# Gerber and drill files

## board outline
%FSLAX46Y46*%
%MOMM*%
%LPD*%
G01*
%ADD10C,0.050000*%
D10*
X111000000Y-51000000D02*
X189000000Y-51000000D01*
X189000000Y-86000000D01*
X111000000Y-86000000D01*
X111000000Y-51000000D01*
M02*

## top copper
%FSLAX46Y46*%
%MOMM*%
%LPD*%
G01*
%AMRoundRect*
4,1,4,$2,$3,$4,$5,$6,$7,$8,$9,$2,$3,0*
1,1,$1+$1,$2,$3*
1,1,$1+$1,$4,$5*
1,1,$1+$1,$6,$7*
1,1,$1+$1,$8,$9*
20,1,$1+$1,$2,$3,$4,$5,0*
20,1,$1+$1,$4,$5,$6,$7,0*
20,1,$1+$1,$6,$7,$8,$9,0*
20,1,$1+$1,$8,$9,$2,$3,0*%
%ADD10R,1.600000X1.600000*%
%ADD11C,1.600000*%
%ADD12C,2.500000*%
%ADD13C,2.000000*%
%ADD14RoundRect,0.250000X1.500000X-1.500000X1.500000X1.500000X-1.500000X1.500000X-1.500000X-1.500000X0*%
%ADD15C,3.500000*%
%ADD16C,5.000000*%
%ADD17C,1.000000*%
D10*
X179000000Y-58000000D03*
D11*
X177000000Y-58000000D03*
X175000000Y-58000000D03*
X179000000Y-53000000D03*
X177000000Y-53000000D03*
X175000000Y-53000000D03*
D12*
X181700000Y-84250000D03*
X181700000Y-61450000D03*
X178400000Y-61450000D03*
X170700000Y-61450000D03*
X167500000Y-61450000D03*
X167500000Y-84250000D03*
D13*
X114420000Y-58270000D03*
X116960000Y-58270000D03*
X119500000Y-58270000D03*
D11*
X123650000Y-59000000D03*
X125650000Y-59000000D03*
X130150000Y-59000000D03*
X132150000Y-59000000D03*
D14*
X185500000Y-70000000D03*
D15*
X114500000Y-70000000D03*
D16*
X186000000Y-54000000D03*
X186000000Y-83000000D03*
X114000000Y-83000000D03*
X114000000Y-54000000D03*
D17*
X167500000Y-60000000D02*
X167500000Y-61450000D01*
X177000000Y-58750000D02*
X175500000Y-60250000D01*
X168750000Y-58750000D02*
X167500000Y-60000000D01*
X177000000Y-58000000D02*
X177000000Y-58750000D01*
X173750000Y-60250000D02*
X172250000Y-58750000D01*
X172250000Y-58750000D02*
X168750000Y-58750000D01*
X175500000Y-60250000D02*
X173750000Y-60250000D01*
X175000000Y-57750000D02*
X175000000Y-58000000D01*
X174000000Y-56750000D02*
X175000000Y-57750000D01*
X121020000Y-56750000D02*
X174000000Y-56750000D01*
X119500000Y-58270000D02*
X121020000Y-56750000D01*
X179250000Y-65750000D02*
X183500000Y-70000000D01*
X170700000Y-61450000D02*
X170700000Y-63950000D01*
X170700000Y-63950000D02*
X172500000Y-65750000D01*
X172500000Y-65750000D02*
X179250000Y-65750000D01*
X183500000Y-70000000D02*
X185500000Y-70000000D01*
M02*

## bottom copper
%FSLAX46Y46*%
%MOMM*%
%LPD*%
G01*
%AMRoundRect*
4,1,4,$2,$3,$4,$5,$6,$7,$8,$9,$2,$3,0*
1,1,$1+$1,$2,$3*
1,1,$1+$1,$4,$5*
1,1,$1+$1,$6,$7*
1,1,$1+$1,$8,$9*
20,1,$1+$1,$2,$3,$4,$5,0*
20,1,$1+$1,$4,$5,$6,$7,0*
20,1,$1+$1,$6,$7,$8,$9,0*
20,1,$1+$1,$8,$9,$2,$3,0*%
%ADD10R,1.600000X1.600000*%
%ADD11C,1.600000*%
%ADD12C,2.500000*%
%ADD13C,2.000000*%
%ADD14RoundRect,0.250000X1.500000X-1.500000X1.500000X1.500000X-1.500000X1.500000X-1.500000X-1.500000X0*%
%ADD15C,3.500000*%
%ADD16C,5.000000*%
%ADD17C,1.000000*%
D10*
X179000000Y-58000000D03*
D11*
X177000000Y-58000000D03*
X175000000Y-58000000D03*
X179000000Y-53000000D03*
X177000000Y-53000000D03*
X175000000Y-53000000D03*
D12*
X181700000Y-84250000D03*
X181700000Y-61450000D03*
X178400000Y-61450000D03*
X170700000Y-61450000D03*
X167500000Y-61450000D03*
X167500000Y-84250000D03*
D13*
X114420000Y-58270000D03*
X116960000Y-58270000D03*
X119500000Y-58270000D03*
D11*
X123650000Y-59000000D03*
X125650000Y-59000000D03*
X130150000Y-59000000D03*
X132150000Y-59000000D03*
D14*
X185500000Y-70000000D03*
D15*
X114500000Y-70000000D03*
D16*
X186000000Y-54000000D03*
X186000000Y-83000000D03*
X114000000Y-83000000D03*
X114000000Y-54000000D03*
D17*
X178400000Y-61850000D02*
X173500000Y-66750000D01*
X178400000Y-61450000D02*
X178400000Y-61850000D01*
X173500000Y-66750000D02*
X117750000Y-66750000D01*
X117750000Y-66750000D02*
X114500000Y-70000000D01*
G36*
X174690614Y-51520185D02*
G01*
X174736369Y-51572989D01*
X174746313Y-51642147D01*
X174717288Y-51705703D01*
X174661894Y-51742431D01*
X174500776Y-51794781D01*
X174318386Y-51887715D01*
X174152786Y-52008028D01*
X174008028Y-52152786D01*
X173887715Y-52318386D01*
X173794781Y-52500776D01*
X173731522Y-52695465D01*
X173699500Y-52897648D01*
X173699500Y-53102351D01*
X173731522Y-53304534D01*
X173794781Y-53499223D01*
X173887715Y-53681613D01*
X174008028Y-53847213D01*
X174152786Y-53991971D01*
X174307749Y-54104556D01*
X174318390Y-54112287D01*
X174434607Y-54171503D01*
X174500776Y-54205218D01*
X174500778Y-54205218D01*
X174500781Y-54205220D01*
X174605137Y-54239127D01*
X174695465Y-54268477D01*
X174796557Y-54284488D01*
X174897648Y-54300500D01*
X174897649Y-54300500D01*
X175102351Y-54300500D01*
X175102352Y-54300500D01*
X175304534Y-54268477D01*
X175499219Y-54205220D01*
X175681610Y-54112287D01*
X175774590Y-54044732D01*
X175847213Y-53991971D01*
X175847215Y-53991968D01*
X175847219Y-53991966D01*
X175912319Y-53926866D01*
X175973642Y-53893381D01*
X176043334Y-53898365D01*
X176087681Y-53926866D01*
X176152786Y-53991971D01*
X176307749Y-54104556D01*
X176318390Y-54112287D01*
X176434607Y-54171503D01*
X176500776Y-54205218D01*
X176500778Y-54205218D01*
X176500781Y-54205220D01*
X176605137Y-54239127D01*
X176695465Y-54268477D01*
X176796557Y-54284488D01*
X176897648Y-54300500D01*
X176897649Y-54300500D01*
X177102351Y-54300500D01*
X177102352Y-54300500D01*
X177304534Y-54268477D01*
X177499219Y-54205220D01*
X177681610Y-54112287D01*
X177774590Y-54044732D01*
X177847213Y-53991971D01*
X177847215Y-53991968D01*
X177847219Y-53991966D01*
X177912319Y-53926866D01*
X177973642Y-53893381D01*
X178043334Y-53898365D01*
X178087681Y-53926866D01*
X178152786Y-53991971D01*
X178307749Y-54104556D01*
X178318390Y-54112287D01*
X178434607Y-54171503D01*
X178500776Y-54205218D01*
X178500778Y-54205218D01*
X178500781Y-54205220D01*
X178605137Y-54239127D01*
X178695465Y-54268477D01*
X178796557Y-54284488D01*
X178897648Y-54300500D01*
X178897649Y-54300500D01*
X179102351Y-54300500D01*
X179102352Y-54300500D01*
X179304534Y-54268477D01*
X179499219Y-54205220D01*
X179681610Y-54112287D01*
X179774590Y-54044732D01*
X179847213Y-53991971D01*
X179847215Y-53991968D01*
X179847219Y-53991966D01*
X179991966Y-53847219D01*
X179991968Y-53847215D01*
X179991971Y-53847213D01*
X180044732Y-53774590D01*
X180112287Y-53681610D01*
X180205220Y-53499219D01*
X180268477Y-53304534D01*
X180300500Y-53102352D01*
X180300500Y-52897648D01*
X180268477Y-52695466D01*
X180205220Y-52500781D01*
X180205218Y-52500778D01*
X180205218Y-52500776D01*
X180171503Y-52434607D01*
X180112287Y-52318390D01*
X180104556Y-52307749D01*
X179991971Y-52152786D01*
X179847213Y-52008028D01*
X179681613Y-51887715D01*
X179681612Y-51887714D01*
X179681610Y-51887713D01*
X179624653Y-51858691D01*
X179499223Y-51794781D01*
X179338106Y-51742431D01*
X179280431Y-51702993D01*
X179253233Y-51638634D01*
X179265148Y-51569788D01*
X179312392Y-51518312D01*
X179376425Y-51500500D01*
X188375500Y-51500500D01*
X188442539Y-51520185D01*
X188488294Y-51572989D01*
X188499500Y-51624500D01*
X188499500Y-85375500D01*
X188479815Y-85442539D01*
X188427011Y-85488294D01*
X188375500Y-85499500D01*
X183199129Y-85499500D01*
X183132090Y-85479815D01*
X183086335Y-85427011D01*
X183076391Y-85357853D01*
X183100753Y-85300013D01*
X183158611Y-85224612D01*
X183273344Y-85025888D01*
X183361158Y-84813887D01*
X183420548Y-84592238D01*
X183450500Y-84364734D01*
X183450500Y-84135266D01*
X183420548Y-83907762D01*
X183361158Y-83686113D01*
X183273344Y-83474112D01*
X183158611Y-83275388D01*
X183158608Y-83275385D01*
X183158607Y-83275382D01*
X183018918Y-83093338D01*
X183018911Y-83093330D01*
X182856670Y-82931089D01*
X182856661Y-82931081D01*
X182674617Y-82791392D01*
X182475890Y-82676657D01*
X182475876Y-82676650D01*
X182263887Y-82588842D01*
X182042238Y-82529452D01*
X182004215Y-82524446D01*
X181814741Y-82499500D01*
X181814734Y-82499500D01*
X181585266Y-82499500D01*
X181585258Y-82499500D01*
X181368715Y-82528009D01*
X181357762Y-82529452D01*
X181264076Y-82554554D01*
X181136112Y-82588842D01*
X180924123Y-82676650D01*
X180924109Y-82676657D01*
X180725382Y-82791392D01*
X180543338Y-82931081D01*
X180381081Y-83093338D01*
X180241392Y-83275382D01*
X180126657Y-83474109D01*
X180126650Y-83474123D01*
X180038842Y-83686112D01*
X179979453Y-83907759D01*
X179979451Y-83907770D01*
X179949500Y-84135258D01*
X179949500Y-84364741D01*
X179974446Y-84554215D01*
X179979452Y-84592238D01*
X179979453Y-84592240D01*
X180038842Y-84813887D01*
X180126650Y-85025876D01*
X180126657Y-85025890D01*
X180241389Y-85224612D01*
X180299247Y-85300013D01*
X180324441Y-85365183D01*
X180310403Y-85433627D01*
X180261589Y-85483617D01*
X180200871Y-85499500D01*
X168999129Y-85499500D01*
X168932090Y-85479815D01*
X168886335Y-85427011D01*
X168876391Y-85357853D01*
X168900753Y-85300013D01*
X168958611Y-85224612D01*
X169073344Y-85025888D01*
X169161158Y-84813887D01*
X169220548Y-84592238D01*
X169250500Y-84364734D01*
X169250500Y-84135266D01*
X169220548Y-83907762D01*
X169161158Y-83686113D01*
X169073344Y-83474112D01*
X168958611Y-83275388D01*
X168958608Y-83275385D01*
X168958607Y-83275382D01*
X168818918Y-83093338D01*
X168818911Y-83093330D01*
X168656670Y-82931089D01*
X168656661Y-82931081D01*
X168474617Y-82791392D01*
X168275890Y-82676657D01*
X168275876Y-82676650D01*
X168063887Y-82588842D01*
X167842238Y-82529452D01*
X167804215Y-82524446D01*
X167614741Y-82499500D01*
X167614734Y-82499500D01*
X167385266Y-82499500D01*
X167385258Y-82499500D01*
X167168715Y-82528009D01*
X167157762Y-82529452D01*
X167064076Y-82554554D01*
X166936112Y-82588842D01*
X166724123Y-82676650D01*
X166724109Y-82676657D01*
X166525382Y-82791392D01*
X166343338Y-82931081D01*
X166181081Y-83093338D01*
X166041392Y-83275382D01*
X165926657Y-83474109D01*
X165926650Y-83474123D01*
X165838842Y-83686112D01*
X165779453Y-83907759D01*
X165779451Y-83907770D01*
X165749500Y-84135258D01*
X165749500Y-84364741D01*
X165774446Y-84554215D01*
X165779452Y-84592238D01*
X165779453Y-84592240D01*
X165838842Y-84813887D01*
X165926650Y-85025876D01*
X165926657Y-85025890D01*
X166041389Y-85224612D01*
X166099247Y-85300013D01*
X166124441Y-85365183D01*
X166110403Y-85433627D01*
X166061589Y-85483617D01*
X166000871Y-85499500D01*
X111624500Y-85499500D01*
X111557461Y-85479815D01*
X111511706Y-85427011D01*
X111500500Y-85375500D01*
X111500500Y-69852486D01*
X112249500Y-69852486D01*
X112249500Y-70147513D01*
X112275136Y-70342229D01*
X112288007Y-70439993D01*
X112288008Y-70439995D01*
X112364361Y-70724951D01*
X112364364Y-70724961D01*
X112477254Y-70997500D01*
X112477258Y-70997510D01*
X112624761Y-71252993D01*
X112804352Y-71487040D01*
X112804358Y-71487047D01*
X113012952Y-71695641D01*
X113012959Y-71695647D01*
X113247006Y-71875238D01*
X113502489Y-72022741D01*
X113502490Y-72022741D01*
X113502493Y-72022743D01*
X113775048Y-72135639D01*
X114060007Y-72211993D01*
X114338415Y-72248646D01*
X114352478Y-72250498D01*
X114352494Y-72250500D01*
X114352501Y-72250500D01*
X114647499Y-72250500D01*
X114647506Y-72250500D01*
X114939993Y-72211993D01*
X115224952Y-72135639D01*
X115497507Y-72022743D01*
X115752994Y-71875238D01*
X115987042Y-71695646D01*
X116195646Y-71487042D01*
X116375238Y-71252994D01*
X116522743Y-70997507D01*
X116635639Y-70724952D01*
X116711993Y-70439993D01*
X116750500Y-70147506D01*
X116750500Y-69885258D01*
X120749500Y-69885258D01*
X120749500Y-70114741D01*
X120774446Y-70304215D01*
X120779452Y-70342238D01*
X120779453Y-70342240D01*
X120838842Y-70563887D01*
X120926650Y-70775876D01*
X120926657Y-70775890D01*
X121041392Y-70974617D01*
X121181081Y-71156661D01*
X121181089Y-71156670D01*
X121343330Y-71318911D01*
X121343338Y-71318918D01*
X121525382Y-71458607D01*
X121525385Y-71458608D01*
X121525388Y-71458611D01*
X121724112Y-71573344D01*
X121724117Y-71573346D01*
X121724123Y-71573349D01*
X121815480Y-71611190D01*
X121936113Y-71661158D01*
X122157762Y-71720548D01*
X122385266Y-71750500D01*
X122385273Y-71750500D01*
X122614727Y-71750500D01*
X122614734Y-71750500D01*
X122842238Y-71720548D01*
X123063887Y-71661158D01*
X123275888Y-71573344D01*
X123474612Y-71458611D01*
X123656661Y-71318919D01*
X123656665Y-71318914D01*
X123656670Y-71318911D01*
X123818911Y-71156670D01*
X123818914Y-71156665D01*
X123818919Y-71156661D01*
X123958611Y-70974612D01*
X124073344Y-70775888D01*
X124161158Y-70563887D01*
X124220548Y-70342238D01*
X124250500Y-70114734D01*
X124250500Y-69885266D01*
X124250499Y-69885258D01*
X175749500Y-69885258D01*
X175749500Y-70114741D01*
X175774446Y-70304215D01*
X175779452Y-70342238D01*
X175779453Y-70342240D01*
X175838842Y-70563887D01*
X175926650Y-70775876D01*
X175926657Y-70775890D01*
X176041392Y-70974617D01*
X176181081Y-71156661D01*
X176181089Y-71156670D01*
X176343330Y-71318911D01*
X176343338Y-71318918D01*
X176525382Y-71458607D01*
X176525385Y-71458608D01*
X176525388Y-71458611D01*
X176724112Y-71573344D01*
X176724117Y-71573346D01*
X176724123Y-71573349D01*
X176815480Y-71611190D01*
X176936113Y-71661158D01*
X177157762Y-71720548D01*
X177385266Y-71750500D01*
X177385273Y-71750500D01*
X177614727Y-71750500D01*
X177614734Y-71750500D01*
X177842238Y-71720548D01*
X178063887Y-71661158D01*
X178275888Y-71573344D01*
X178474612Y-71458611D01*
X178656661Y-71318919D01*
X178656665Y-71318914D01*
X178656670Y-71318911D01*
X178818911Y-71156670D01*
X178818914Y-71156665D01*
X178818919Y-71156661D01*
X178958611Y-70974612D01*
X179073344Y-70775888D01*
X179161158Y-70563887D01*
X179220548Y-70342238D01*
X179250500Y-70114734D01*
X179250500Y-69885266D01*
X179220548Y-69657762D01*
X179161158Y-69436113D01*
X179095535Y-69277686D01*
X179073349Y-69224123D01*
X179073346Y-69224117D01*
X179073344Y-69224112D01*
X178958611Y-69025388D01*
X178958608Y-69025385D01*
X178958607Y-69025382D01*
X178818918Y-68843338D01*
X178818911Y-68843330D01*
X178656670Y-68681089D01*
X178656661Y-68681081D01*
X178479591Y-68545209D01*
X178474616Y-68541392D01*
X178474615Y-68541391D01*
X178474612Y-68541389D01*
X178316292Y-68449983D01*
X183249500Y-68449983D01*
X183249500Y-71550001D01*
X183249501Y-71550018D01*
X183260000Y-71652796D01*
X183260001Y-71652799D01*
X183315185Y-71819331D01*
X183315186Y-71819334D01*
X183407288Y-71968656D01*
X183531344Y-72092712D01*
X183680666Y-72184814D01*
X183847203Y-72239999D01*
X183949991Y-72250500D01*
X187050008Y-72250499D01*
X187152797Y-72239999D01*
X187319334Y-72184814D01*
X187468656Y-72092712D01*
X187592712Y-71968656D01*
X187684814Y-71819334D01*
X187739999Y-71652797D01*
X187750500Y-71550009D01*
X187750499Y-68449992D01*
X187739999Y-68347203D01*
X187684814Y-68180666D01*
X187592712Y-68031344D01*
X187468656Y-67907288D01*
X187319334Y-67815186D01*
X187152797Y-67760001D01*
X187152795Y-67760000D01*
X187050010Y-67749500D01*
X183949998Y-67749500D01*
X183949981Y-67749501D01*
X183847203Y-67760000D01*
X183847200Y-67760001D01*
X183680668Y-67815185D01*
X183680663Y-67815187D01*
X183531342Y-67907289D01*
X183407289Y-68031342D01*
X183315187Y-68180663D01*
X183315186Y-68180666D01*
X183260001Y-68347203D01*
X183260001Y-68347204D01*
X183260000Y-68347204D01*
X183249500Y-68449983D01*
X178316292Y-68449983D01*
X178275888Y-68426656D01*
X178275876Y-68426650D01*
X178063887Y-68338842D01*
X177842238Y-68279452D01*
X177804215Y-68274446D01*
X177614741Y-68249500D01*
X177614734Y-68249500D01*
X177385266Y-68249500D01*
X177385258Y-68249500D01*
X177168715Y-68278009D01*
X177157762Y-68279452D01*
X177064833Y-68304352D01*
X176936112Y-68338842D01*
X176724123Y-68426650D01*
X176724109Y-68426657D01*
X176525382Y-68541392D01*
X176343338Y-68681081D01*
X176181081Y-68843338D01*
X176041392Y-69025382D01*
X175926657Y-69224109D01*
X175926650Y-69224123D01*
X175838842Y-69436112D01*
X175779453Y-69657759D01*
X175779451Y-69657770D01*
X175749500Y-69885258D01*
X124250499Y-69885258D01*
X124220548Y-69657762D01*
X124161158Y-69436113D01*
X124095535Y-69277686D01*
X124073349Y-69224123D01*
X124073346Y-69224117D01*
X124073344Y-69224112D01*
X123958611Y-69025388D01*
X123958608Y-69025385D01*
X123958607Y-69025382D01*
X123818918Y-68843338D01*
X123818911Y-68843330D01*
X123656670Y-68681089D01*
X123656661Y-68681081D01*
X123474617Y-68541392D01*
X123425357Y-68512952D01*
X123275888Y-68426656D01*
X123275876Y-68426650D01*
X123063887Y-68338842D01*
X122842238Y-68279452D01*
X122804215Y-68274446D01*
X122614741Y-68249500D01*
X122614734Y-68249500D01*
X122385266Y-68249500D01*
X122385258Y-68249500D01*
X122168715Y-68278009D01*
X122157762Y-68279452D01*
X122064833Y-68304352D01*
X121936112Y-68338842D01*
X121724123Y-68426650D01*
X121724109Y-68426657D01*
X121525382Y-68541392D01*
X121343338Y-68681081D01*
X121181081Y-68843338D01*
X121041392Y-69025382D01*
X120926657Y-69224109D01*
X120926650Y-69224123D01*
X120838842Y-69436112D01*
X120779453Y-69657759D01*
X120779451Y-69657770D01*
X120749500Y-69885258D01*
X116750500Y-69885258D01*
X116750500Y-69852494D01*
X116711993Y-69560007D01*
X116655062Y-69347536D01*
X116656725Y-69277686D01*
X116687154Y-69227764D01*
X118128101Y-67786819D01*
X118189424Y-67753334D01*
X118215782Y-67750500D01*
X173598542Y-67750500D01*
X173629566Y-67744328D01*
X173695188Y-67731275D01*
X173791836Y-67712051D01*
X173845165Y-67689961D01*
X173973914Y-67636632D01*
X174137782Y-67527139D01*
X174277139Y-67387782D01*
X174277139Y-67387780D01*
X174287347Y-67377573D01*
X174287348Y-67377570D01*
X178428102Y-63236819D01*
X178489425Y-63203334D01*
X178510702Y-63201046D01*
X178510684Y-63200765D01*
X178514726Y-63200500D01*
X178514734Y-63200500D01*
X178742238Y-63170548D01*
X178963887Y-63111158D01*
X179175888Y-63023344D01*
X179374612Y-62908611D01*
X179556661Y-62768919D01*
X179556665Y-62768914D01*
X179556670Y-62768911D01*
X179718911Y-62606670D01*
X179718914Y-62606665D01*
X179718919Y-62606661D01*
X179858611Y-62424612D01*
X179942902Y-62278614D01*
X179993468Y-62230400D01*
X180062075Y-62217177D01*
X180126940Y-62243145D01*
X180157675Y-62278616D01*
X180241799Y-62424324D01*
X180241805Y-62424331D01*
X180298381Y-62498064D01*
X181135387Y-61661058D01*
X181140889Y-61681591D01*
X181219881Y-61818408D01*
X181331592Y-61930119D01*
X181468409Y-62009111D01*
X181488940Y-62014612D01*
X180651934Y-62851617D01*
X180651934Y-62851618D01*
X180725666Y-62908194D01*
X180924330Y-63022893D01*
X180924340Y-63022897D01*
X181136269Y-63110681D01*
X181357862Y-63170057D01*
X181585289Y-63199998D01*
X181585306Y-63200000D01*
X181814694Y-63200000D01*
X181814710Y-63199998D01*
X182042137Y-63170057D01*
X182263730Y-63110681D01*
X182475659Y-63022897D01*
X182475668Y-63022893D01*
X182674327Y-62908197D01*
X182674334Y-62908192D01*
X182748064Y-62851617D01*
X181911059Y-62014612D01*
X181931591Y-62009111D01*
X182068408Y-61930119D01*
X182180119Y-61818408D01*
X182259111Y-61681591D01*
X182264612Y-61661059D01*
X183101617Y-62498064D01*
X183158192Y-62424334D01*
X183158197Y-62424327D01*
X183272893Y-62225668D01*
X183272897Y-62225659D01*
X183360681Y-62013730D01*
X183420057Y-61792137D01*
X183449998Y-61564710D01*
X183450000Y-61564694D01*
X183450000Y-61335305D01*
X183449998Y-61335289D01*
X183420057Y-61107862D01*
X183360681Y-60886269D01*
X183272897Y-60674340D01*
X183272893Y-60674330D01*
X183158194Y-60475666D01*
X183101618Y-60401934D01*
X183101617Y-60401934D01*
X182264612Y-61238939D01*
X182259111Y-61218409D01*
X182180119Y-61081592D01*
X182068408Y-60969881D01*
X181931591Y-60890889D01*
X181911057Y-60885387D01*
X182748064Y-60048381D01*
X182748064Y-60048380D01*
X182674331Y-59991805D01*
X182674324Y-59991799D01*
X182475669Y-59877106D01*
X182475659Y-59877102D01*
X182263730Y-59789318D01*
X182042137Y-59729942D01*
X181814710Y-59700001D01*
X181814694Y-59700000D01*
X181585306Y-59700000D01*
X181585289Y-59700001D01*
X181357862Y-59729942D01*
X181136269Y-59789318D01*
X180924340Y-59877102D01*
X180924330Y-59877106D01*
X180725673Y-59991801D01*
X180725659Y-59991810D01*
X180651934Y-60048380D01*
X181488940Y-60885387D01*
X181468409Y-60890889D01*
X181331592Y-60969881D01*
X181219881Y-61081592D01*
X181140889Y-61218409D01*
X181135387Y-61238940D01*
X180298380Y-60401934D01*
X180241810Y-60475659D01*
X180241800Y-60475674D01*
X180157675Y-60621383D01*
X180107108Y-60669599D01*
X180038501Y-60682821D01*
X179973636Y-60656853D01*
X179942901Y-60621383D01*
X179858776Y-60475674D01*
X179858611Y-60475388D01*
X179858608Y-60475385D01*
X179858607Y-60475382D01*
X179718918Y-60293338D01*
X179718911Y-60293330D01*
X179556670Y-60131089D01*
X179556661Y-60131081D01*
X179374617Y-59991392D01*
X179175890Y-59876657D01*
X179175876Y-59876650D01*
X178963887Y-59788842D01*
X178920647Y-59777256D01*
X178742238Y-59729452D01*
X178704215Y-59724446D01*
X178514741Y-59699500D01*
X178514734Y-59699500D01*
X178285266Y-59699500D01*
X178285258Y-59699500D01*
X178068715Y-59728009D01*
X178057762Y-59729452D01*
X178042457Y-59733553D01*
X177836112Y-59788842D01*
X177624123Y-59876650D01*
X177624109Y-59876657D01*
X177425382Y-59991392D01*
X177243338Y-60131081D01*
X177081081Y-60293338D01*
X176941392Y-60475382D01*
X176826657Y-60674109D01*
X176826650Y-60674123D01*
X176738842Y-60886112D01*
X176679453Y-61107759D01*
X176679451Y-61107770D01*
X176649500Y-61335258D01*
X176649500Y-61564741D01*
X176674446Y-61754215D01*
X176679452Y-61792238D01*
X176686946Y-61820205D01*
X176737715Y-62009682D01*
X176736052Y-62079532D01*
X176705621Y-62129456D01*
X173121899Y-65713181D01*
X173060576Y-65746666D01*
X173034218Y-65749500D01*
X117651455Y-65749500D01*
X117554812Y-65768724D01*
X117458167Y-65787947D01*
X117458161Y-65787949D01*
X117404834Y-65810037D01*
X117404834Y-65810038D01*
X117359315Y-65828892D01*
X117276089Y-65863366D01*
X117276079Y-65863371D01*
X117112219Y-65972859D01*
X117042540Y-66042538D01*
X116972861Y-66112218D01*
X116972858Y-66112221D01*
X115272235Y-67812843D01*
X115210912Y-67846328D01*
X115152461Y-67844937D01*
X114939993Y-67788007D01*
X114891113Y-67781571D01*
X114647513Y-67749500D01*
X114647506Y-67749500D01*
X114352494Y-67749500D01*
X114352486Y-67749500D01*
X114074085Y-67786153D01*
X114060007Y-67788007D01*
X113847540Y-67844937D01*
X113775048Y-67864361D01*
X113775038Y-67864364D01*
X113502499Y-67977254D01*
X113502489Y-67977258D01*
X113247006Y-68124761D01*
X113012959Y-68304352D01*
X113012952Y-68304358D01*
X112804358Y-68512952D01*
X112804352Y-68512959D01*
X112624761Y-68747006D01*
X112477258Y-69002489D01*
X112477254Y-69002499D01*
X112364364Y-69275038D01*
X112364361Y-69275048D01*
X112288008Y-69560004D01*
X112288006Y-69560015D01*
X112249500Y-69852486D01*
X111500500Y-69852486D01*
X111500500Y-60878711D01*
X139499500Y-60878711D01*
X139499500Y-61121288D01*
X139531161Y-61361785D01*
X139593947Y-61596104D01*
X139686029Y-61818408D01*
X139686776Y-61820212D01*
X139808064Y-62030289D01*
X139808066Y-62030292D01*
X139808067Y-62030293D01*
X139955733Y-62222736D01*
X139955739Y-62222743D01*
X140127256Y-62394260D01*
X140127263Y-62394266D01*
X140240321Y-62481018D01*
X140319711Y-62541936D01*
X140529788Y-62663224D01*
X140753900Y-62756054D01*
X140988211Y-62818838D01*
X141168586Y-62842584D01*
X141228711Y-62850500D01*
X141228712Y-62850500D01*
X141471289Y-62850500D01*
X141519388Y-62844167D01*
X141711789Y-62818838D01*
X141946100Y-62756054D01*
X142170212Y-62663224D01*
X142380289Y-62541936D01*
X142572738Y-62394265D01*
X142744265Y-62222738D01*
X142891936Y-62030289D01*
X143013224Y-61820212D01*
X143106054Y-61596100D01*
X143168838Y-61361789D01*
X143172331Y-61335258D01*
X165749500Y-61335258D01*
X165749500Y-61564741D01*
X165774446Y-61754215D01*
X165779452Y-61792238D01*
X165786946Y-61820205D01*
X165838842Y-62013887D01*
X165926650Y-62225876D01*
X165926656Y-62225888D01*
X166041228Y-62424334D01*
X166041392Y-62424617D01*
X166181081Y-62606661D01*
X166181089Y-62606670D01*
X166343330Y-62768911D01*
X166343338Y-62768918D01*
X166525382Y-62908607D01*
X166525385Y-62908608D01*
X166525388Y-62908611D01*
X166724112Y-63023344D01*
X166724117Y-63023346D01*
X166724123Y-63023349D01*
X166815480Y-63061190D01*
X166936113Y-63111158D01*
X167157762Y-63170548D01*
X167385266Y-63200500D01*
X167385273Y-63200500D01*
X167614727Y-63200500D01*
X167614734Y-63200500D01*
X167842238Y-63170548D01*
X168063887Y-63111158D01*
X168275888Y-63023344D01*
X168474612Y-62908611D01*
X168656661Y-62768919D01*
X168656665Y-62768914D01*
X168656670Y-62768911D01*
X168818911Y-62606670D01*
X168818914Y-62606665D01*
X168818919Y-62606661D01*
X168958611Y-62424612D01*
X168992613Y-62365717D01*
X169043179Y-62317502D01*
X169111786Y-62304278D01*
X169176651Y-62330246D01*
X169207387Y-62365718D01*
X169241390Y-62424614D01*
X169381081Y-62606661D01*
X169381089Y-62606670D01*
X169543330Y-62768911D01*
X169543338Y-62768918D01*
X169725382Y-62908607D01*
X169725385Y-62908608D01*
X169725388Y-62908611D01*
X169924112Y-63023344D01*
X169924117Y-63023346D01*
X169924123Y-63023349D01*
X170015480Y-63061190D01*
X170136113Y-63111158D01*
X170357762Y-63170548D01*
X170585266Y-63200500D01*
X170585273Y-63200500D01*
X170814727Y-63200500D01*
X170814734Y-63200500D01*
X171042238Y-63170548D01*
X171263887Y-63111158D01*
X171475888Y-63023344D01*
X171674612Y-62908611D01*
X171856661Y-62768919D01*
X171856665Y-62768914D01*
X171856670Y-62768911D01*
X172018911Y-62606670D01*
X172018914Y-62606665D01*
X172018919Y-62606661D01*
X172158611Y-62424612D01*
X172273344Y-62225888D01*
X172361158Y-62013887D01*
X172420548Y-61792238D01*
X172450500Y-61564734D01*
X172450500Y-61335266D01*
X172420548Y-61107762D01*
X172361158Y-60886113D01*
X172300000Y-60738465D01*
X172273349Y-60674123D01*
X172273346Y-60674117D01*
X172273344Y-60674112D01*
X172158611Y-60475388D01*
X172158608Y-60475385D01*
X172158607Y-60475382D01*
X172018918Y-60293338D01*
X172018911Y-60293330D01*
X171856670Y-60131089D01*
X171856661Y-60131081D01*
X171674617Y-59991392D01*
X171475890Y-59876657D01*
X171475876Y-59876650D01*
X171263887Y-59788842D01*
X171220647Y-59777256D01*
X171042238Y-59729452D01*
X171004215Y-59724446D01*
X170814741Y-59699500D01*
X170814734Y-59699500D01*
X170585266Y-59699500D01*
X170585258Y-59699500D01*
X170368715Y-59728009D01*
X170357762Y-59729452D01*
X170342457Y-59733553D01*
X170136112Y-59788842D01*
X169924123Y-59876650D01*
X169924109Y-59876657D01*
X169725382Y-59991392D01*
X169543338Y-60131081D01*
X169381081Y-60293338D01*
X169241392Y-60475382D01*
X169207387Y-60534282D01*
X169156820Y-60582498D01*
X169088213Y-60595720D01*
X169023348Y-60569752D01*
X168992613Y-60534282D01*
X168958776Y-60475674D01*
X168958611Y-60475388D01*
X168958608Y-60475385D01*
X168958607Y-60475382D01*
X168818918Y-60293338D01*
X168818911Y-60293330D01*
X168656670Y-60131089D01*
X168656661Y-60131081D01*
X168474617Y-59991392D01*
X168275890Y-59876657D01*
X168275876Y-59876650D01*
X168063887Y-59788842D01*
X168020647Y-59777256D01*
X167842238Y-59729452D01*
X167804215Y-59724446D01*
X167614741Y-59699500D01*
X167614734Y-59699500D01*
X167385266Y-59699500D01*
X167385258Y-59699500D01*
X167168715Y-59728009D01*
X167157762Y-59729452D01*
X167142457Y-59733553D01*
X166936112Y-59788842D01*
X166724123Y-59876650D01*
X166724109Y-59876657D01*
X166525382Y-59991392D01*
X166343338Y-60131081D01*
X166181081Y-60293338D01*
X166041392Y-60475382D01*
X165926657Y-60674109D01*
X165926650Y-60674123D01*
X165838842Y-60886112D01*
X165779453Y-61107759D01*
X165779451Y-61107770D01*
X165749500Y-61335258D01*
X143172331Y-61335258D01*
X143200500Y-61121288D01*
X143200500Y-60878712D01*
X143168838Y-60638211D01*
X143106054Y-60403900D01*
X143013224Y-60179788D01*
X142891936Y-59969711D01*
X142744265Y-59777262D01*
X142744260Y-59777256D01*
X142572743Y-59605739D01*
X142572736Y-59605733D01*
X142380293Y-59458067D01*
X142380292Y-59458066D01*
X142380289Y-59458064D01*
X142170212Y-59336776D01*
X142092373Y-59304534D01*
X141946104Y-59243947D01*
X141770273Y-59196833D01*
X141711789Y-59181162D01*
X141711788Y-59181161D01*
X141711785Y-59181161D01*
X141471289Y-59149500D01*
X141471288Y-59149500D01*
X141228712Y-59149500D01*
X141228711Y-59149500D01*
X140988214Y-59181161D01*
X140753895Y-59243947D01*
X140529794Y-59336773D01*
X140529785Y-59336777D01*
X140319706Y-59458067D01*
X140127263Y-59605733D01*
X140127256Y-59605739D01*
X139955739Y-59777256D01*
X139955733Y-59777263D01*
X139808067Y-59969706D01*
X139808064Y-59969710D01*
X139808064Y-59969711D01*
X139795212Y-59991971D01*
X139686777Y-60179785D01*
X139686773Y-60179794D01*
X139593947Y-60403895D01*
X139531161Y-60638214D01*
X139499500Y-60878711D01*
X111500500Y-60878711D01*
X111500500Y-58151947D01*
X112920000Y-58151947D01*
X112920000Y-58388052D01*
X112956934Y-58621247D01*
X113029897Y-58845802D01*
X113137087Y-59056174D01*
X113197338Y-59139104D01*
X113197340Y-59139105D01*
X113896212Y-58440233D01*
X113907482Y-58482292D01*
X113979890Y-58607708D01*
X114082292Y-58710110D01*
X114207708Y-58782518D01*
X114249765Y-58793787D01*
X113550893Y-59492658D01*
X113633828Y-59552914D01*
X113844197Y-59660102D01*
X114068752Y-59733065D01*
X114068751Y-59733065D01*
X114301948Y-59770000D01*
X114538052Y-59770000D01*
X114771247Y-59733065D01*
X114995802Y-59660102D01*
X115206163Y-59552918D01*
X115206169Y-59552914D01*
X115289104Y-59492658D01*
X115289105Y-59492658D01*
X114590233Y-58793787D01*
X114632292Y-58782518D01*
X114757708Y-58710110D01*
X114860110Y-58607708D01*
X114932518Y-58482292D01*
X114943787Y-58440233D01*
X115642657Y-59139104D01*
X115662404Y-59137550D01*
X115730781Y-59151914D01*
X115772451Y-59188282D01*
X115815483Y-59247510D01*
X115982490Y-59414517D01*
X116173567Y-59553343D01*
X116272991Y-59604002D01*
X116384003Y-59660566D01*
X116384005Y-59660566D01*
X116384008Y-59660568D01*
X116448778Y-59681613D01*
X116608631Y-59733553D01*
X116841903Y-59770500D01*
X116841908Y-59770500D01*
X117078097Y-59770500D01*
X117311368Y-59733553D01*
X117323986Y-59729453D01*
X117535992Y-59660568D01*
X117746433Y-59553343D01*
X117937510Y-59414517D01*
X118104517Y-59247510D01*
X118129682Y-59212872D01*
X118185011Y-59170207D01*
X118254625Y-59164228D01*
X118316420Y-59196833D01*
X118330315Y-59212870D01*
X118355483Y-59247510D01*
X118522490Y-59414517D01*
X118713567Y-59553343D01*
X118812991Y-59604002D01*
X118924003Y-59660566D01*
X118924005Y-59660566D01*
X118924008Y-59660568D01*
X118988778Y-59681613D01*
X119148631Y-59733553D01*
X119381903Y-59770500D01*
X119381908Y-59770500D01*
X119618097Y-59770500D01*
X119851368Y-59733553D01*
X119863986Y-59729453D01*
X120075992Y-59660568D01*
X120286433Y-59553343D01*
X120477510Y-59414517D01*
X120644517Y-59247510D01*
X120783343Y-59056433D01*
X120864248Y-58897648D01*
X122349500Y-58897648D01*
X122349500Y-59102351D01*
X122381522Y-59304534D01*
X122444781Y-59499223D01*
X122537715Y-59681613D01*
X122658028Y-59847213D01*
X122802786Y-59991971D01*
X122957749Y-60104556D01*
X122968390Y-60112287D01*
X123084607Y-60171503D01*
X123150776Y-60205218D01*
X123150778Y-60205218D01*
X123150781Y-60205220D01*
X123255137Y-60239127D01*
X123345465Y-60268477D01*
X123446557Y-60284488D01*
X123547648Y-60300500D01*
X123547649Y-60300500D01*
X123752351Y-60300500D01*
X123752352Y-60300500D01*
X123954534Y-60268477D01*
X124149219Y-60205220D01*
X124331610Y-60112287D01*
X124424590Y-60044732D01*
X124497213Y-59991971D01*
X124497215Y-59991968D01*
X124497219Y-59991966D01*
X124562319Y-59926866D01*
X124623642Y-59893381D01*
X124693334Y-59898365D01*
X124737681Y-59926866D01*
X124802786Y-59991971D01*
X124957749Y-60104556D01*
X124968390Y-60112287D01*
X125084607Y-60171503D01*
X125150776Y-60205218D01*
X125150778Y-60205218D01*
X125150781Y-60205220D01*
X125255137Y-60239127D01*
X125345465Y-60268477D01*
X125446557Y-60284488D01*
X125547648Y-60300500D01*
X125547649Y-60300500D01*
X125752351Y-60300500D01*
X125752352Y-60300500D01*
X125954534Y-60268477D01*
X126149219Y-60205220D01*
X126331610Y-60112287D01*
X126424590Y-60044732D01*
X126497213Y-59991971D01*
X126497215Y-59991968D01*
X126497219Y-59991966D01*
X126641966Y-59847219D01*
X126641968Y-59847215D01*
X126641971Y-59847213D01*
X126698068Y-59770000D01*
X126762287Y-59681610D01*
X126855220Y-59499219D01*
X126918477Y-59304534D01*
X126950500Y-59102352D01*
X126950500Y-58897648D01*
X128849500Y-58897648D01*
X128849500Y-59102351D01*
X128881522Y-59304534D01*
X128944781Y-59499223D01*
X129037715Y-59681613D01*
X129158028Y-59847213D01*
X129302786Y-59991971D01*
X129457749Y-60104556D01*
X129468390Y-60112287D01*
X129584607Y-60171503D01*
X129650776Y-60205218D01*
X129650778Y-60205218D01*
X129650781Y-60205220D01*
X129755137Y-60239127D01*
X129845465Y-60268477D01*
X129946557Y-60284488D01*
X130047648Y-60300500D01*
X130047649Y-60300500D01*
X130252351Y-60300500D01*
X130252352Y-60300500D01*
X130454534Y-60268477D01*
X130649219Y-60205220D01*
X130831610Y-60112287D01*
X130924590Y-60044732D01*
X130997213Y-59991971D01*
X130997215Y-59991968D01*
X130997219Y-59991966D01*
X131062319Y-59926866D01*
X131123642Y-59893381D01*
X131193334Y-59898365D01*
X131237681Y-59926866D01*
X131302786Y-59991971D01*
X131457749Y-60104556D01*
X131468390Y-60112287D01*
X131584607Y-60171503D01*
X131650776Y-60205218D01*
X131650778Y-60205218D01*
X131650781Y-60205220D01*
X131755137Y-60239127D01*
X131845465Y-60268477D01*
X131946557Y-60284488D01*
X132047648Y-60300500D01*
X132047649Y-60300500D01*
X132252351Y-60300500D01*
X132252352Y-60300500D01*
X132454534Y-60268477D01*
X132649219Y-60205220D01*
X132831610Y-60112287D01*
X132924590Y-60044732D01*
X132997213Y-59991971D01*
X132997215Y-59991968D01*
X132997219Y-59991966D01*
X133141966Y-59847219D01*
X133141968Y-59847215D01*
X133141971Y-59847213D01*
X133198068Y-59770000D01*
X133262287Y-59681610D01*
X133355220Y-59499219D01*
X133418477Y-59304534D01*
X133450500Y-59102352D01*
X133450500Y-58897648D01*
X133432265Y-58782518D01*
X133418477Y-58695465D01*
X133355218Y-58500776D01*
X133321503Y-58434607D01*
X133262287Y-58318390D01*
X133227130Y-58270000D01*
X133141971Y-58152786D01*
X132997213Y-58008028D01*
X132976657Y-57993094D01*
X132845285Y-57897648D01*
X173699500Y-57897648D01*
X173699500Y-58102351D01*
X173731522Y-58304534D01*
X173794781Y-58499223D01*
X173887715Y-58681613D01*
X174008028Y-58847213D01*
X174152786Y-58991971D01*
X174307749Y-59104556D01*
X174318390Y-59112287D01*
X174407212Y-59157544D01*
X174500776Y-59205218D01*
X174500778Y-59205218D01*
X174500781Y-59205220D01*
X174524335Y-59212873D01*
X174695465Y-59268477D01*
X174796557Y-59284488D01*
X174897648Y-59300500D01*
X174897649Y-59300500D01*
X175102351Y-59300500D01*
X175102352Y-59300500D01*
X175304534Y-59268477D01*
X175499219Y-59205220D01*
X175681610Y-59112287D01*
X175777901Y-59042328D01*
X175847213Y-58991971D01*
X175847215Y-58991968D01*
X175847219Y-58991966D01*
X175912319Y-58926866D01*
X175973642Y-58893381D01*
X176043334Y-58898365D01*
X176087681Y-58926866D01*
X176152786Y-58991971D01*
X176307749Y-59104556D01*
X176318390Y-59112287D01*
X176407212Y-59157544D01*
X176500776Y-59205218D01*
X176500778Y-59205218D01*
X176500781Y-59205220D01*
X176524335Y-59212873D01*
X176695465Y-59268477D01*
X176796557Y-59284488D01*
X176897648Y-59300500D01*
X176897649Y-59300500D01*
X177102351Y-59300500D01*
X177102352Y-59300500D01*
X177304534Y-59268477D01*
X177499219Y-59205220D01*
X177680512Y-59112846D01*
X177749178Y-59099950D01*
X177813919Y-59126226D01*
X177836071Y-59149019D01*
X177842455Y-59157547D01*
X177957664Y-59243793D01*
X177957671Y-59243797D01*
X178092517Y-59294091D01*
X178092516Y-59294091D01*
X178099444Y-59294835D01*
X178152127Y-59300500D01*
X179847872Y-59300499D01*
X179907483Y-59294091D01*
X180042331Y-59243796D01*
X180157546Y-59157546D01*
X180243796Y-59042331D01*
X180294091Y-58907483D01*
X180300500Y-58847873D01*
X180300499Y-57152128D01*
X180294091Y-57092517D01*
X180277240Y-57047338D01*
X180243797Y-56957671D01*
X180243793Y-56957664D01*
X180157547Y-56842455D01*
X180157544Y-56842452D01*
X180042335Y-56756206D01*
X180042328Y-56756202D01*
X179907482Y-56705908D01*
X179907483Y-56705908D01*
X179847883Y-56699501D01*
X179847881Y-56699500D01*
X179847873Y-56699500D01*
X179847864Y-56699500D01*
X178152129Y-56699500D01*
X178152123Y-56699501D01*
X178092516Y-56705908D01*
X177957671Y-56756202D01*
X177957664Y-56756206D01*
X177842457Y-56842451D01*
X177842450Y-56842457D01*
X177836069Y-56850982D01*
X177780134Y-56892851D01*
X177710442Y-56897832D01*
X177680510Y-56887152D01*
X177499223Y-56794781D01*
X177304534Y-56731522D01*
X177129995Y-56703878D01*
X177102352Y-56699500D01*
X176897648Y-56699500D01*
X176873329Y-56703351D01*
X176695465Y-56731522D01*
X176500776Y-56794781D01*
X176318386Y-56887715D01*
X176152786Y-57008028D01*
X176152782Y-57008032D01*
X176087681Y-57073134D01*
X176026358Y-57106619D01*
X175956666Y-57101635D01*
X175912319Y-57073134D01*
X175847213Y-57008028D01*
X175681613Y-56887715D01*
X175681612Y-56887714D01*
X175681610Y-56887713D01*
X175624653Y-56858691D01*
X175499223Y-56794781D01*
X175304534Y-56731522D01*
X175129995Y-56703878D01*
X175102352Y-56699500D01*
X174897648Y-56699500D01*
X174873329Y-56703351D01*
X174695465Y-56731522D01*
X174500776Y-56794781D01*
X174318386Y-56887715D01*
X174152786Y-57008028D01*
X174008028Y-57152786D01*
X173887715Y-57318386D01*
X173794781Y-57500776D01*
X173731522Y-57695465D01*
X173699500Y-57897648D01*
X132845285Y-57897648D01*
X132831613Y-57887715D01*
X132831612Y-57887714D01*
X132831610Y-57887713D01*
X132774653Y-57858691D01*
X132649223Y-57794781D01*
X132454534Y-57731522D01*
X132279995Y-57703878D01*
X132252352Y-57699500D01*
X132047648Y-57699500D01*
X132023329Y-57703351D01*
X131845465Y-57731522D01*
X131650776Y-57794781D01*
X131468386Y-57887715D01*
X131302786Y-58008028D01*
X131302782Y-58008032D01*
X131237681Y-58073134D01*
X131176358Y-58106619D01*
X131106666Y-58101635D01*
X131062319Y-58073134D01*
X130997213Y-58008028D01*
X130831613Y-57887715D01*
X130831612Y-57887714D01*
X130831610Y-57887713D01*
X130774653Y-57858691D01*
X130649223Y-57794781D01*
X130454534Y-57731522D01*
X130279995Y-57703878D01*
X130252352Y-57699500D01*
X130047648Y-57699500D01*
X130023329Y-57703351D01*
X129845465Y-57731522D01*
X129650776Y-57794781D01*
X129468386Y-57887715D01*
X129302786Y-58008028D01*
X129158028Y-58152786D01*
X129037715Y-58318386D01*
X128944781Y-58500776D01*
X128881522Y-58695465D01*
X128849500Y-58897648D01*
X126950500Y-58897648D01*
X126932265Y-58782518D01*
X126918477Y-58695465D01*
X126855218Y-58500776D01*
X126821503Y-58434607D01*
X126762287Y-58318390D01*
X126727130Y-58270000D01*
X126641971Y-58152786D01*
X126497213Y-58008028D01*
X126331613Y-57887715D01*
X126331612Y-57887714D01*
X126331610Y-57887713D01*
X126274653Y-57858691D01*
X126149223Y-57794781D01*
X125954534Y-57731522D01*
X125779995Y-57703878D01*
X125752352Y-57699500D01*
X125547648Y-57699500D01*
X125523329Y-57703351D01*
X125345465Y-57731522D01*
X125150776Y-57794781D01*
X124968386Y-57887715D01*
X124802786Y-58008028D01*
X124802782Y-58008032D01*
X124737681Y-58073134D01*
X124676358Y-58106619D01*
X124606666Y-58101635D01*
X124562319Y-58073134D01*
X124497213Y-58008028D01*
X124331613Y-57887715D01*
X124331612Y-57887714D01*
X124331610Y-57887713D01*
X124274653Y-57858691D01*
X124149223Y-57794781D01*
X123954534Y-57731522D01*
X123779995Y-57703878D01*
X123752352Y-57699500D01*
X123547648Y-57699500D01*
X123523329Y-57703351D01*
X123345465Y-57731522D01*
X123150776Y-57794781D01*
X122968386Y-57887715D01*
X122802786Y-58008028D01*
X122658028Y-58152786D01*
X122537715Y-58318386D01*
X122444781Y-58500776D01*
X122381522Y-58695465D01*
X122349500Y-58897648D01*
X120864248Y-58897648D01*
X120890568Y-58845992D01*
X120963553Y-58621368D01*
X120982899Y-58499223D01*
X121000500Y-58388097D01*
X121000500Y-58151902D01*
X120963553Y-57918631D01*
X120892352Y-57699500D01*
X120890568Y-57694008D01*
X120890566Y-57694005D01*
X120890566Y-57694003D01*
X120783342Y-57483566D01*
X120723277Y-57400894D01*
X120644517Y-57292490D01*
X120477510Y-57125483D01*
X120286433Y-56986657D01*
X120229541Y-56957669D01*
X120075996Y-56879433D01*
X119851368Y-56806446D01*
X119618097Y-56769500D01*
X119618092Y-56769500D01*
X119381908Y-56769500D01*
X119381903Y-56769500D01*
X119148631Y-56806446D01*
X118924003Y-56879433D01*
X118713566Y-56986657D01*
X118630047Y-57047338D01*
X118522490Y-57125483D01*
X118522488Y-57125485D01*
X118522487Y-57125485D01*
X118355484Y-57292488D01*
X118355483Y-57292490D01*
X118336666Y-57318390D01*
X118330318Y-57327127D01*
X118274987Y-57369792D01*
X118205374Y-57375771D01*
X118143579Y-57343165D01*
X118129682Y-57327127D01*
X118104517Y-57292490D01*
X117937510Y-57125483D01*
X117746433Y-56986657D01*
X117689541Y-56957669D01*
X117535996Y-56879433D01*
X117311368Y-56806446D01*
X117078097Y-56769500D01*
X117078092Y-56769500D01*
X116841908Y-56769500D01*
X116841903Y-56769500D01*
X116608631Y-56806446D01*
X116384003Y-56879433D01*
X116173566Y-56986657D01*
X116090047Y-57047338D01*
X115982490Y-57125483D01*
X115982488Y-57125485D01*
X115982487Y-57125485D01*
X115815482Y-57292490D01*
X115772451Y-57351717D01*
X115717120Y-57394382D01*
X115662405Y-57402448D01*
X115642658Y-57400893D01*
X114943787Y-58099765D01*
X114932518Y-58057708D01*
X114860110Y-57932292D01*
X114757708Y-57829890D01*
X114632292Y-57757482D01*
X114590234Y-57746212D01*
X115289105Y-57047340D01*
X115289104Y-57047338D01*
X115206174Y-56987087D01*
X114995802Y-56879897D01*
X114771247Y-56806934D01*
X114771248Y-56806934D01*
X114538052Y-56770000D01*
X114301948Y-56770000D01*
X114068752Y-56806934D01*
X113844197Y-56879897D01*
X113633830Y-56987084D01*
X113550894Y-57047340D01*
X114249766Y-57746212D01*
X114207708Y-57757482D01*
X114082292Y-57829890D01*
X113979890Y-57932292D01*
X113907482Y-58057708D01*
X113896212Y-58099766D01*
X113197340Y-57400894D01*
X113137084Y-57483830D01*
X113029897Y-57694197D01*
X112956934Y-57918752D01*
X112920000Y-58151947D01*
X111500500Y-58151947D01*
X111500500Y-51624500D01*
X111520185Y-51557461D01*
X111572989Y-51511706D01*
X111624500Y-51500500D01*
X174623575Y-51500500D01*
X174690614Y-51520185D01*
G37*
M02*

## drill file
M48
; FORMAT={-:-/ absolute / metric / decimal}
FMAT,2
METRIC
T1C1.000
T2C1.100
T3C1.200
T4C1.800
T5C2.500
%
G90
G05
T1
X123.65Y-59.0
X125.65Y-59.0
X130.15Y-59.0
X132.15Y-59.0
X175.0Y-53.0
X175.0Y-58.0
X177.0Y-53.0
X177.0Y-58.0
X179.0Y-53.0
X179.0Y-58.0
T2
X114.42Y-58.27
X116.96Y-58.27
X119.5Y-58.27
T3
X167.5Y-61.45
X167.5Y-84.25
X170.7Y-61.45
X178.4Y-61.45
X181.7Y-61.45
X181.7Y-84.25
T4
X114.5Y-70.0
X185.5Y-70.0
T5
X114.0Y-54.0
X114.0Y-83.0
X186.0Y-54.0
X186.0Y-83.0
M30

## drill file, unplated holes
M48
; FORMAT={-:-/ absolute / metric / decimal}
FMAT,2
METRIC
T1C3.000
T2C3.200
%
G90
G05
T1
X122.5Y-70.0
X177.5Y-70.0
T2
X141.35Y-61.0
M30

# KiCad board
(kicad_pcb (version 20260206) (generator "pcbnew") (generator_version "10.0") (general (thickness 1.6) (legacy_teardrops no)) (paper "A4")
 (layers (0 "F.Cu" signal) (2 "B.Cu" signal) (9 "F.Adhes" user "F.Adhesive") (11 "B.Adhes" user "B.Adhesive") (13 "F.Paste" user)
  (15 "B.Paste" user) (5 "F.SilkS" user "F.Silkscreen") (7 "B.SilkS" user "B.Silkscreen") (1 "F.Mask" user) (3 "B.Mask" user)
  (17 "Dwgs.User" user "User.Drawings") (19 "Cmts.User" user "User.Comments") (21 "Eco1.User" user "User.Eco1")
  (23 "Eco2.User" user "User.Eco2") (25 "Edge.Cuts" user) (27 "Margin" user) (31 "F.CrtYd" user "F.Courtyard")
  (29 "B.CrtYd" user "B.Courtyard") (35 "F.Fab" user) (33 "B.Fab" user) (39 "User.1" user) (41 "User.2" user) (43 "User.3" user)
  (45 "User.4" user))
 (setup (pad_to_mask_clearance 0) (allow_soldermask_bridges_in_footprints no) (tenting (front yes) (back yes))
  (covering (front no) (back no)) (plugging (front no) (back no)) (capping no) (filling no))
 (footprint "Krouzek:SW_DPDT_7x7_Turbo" (layer "F.Cu") (at 177 55.5 180)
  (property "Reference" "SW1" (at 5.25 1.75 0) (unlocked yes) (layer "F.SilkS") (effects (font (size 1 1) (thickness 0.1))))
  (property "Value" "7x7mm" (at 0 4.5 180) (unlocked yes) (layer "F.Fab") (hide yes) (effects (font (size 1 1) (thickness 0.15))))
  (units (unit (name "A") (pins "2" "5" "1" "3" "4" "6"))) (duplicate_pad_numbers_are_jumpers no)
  (pad "1" thru_hole rect (at -2 -2.5 180) (size 1.6 1.6) (drill 1) (layers "*.Cu" "*.Mask") (remove_unused_layers no)
   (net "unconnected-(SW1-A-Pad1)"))
  (pad "2" thru_hole circle (at 0 -2.5 180) (size 1.6 1.6) (drill 1) (layers "*.Cu" "*.Mask") (remove_unused_layers no)
   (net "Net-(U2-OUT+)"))
  (pad "3" thru_hole circle (at 2 -2.5 180) (size 1.6 1.6) (drill 1) (layers "*.Cu" "*.Mask") (remove_unused_layers no)
   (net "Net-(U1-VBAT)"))
  (pad "4" thru_hole circle (at -2 2.5 180) (size 1.6 1.6) (drill 1) (layers "*.Cu" "*.Mask") (remove_unused_layers no)
   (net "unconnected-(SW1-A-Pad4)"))
  (pad "5" thru_hole circle (at 0 2.5 180) (size 1.6 1.6) (drill 1) (layers "*.Cu" "*.Mask") (remove_unused_layers no)
   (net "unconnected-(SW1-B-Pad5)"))
  (pad "6" thru_hole circle (at 2 2.5 180) (size 1.6 1.6) (drill 1) (layers "*.Cu" "*.Mask") (remove_unused_layers no)
   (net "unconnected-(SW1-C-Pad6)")))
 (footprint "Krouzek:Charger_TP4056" (layer "F.Cu") (at 166 86.05 90)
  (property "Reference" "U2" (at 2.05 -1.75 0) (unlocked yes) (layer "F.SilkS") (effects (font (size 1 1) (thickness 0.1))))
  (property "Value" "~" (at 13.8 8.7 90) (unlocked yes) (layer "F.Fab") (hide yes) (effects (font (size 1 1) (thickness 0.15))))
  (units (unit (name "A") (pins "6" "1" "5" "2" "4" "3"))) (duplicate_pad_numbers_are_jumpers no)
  (pad "1" thru_hole circle (at 1.8 15.7 180) (size 2.5 2.5) (drill 1.2) (layers "*.Cu" "*.Mask") (remove_unused_layers no)
   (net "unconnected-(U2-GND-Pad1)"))
  (pad "2" thru_hole circle (at 24.6 15.7 180) (size 2.5 2.5) (drill 1.2) (layers "*.Cu" "*.Mask") (remove_unused_layers no) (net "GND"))
  (pad "3" thru_hole circle (at 24.6 12.4 180) (size 2.5 2.5) (drill 1.2) (layers "*.Cu" "*.Mask") (remove_unused_layers no)
   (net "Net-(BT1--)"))
  (pad "4" thru_hole circle (at 24.6 4.7 180) (size 2.5 2.5) (drill 1.2) (layers "*.Cu" "*.Mask") (remove_unused_layers no)
   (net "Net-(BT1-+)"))
  (pad "5" thru_hole circle (at 24.6 1.5 180) (size 2.5 2.5) (drill 1.2) (layers "*.Cu" "*.Mask") (remove_unused_layers no)
   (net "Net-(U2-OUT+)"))
  (pad "6" thru_hole circle (at 1.8 1.5 180) (size 2.5 2.5) (drill 1.2) (layers "*.Cu" "*.Mask") (remove_unused_layers no)
   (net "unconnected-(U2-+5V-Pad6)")))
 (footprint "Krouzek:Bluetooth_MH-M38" (layer "F.Cu") (at 113.15 57)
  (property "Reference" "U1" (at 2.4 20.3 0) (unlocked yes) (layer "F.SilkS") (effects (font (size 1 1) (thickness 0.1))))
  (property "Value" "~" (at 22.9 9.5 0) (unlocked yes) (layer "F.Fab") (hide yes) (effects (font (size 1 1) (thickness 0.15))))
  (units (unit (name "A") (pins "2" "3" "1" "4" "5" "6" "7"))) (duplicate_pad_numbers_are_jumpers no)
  (pad "" np_thru_hole circle (at 28.2 4 90) (size 3.2 3.2) (drill 3.2) (layers "*.Cu" "*.Mask"))
  (pad "1" thru_hole circle (at 1.27 1.27 90) (size 2 2) (drill 1.1) (layers "*.Cu" "*.Mask") (remove_unused_layers no) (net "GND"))
  (pad "2" thru_hole circle (at 3.81 1.27 90) (size 2 2) (drill 1.1) (layers "*.Cu" "*.Mask") (remove_unused_layers no)
   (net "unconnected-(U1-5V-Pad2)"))
  (pad "3" thru_hole circle (at 6.35 1.27 90) (size 2 2) (drill 1.1) (layers "*.Cu" "*.Mask") (remove_unused_layers no)
   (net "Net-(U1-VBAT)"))
  (pad "4" thru_hole circle (at 10.5 2 90) (size 1.6 1.6) (drill 1) (layers "*.Cu" "*.Mask") (remove_unused_layers no)
   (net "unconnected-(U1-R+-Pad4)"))
  (pad "5" thru_hole circle (at 12.5 2 90) (size 1.6 1.6) (drill 1) (layers "*.Cu" "*.Mask") (remove_unused_layers no)
   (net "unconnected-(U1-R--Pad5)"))
  (pad "6" thru_hole circle (at 17 2 90) (size 1.6 1.6) (drill 1) (layers "*.Cu" "*.Mask") (remove_unused_layers no)
   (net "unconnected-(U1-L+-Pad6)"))
  (pad "7" thru_hole circle (at 19 2 90) (size 1.6 1.6) (drill 1) (layers "*.Cu" "*.Mask") (remove_unused_layers no)
   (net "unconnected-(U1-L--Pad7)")))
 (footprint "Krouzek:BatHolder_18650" (layer "B.Cu") (at 188.5 59.5 180)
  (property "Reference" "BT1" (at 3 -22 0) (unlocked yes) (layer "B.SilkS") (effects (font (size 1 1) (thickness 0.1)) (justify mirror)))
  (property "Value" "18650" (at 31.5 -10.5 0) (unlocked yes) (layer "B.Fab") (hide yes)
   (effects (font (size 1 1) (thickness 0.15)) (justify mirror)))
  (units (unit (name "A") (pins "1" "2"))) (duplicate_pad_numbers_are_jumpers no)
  (pad "" np_thru_hole circle (at 11 -10.5 90) (size 3 3) (drill 3) (layers "*.Cu" "*.Mask"))
  (pad "" np_thru_hole circle (at 66 -10.5 90) (size 3 3) (drill 3) (layers "*.Cu" "*.Mask"))
  (pad "1" thru_hole roundrect (at 3 -10.5 90) (size 3.5 3.5) (drill 1.8) (layers "*.Cu" "*.Mask") (remove_unused_layers no)
   (roundrect_rratio 0.07142857143) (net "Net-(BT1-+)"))
  (pad "2" thru_hole circle (at 74 -10.5 90) (size 3.5 3.5) (drill 1.8) (layers "*.Cu" "*.Mask") (remove_unused_layers no)
   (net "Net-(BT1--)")))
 (gr_rect (start 111 51) (end 189 86) (stroke (width 0.05) (type default)) (fill no) (layer "Edge.Cuts"))
 (segment (start 167.5 60) (end 167.5 61.45) (width 1) (layer "F.Cu") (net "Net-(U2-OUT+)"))
 (segment (start 177 58.75) (end 175.5 60.25) (width 1) (layer "F.Cu") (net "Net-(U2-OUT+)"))
 (segment (start 168.75 58.75) (end 167.5 60) (width 1) (layer "F.Cu") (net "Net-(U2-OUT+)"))
 (segment (start 177 58) (end 177 58.75) (width 1) (layer "F.Cu") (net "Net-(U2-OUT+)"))
 (segment (start 173.75 60.25) (end 172.25 58.75) (width 1) (layer "F.Cu") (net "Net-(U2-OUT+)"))
 (segment (start 172.25 58.75) (end 168.75 58.75) (width 1) (layer "F.Cu") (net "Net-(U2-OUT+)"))
 (segment (start 175.5 60.25) (end 173.75 60.25) (width 1) (layer "F.Cu") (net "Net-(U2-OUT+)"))
 (segment (start 175 57.75) (end 175 58) (width 1) (layer "F.Cu") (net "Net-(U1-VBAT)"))
 (segment (start 174 56.75) (end 175 57.75) (width 1) (layer "F.Cu") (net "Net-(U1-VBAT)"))
 (segment (start 121.02 56.75) (end 174 56.75) (width 1) (layer "F.Cu") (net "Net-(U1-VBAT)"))
 (segment (start 119.5 58.27) (end 121.02 56.75) (width 1) (layer "F.Cu") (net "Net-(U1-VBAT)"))
 (via (at 186 54) (size 5) (drill 2.5) (layers "F.Cu" "B.Cu") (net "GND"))
 (via (at 186 83) (size 5) (drill 2.5) (layers "F.Cu" "B.Cu") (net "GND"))
 (via (at 114 83) (size 5) (drill 2.5) (layers "F.Cu" "B.Cu") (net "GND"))
 (via (at 114 54) (size 5) (drill 2.5) (layers "F.Cu" "B.Cu") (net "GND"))
 (segment (start 178.4 61.85) (end 173.5 66.75) (width 1) (layer "B.Cu") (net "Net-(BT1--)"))
 (segment (start 178.4 61.45) (end 178.4 61.85) (width 1) (layer "B.Cu") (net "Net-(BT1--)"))
 (segment (start 173.5 66.75) (end 117.75 66.75) (width 1) (layer "B.Cu") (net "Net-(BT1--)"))
 (segment (start 117.75 66.75) (end 114.5 70) (width 1) (layer "B.Cu") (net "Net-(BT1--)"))
 (segment (start 179.25 65.75) (end 183.5 70) (width 1) (layer "F.Cu") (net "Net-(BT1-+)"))
 (segment (start 170.7 61.45) (end 170.7 63.95) (width 1) (layer "F.Cu") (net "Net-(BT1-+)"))
 (segment (start 170.7 63.95) (end 172.5 65.75) (width 1) (layer "F.Cu") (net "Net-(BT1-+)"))
 (segment (start 172.5 65.75) (end 179.25 65.75) (width 1) (layer "F.Cu") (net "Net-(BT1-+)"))
 (segment (start 183.5 70) (end 185.5 70) (width 1) (layer "F.Cu") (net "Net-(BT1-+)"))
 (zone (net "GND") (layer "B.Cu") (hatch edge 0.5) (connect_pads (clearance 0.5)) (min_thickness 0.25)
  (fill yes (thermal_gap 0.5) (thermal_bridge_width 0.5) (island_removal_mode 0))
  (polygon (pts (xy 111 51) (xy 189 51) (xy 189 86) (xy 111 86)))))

